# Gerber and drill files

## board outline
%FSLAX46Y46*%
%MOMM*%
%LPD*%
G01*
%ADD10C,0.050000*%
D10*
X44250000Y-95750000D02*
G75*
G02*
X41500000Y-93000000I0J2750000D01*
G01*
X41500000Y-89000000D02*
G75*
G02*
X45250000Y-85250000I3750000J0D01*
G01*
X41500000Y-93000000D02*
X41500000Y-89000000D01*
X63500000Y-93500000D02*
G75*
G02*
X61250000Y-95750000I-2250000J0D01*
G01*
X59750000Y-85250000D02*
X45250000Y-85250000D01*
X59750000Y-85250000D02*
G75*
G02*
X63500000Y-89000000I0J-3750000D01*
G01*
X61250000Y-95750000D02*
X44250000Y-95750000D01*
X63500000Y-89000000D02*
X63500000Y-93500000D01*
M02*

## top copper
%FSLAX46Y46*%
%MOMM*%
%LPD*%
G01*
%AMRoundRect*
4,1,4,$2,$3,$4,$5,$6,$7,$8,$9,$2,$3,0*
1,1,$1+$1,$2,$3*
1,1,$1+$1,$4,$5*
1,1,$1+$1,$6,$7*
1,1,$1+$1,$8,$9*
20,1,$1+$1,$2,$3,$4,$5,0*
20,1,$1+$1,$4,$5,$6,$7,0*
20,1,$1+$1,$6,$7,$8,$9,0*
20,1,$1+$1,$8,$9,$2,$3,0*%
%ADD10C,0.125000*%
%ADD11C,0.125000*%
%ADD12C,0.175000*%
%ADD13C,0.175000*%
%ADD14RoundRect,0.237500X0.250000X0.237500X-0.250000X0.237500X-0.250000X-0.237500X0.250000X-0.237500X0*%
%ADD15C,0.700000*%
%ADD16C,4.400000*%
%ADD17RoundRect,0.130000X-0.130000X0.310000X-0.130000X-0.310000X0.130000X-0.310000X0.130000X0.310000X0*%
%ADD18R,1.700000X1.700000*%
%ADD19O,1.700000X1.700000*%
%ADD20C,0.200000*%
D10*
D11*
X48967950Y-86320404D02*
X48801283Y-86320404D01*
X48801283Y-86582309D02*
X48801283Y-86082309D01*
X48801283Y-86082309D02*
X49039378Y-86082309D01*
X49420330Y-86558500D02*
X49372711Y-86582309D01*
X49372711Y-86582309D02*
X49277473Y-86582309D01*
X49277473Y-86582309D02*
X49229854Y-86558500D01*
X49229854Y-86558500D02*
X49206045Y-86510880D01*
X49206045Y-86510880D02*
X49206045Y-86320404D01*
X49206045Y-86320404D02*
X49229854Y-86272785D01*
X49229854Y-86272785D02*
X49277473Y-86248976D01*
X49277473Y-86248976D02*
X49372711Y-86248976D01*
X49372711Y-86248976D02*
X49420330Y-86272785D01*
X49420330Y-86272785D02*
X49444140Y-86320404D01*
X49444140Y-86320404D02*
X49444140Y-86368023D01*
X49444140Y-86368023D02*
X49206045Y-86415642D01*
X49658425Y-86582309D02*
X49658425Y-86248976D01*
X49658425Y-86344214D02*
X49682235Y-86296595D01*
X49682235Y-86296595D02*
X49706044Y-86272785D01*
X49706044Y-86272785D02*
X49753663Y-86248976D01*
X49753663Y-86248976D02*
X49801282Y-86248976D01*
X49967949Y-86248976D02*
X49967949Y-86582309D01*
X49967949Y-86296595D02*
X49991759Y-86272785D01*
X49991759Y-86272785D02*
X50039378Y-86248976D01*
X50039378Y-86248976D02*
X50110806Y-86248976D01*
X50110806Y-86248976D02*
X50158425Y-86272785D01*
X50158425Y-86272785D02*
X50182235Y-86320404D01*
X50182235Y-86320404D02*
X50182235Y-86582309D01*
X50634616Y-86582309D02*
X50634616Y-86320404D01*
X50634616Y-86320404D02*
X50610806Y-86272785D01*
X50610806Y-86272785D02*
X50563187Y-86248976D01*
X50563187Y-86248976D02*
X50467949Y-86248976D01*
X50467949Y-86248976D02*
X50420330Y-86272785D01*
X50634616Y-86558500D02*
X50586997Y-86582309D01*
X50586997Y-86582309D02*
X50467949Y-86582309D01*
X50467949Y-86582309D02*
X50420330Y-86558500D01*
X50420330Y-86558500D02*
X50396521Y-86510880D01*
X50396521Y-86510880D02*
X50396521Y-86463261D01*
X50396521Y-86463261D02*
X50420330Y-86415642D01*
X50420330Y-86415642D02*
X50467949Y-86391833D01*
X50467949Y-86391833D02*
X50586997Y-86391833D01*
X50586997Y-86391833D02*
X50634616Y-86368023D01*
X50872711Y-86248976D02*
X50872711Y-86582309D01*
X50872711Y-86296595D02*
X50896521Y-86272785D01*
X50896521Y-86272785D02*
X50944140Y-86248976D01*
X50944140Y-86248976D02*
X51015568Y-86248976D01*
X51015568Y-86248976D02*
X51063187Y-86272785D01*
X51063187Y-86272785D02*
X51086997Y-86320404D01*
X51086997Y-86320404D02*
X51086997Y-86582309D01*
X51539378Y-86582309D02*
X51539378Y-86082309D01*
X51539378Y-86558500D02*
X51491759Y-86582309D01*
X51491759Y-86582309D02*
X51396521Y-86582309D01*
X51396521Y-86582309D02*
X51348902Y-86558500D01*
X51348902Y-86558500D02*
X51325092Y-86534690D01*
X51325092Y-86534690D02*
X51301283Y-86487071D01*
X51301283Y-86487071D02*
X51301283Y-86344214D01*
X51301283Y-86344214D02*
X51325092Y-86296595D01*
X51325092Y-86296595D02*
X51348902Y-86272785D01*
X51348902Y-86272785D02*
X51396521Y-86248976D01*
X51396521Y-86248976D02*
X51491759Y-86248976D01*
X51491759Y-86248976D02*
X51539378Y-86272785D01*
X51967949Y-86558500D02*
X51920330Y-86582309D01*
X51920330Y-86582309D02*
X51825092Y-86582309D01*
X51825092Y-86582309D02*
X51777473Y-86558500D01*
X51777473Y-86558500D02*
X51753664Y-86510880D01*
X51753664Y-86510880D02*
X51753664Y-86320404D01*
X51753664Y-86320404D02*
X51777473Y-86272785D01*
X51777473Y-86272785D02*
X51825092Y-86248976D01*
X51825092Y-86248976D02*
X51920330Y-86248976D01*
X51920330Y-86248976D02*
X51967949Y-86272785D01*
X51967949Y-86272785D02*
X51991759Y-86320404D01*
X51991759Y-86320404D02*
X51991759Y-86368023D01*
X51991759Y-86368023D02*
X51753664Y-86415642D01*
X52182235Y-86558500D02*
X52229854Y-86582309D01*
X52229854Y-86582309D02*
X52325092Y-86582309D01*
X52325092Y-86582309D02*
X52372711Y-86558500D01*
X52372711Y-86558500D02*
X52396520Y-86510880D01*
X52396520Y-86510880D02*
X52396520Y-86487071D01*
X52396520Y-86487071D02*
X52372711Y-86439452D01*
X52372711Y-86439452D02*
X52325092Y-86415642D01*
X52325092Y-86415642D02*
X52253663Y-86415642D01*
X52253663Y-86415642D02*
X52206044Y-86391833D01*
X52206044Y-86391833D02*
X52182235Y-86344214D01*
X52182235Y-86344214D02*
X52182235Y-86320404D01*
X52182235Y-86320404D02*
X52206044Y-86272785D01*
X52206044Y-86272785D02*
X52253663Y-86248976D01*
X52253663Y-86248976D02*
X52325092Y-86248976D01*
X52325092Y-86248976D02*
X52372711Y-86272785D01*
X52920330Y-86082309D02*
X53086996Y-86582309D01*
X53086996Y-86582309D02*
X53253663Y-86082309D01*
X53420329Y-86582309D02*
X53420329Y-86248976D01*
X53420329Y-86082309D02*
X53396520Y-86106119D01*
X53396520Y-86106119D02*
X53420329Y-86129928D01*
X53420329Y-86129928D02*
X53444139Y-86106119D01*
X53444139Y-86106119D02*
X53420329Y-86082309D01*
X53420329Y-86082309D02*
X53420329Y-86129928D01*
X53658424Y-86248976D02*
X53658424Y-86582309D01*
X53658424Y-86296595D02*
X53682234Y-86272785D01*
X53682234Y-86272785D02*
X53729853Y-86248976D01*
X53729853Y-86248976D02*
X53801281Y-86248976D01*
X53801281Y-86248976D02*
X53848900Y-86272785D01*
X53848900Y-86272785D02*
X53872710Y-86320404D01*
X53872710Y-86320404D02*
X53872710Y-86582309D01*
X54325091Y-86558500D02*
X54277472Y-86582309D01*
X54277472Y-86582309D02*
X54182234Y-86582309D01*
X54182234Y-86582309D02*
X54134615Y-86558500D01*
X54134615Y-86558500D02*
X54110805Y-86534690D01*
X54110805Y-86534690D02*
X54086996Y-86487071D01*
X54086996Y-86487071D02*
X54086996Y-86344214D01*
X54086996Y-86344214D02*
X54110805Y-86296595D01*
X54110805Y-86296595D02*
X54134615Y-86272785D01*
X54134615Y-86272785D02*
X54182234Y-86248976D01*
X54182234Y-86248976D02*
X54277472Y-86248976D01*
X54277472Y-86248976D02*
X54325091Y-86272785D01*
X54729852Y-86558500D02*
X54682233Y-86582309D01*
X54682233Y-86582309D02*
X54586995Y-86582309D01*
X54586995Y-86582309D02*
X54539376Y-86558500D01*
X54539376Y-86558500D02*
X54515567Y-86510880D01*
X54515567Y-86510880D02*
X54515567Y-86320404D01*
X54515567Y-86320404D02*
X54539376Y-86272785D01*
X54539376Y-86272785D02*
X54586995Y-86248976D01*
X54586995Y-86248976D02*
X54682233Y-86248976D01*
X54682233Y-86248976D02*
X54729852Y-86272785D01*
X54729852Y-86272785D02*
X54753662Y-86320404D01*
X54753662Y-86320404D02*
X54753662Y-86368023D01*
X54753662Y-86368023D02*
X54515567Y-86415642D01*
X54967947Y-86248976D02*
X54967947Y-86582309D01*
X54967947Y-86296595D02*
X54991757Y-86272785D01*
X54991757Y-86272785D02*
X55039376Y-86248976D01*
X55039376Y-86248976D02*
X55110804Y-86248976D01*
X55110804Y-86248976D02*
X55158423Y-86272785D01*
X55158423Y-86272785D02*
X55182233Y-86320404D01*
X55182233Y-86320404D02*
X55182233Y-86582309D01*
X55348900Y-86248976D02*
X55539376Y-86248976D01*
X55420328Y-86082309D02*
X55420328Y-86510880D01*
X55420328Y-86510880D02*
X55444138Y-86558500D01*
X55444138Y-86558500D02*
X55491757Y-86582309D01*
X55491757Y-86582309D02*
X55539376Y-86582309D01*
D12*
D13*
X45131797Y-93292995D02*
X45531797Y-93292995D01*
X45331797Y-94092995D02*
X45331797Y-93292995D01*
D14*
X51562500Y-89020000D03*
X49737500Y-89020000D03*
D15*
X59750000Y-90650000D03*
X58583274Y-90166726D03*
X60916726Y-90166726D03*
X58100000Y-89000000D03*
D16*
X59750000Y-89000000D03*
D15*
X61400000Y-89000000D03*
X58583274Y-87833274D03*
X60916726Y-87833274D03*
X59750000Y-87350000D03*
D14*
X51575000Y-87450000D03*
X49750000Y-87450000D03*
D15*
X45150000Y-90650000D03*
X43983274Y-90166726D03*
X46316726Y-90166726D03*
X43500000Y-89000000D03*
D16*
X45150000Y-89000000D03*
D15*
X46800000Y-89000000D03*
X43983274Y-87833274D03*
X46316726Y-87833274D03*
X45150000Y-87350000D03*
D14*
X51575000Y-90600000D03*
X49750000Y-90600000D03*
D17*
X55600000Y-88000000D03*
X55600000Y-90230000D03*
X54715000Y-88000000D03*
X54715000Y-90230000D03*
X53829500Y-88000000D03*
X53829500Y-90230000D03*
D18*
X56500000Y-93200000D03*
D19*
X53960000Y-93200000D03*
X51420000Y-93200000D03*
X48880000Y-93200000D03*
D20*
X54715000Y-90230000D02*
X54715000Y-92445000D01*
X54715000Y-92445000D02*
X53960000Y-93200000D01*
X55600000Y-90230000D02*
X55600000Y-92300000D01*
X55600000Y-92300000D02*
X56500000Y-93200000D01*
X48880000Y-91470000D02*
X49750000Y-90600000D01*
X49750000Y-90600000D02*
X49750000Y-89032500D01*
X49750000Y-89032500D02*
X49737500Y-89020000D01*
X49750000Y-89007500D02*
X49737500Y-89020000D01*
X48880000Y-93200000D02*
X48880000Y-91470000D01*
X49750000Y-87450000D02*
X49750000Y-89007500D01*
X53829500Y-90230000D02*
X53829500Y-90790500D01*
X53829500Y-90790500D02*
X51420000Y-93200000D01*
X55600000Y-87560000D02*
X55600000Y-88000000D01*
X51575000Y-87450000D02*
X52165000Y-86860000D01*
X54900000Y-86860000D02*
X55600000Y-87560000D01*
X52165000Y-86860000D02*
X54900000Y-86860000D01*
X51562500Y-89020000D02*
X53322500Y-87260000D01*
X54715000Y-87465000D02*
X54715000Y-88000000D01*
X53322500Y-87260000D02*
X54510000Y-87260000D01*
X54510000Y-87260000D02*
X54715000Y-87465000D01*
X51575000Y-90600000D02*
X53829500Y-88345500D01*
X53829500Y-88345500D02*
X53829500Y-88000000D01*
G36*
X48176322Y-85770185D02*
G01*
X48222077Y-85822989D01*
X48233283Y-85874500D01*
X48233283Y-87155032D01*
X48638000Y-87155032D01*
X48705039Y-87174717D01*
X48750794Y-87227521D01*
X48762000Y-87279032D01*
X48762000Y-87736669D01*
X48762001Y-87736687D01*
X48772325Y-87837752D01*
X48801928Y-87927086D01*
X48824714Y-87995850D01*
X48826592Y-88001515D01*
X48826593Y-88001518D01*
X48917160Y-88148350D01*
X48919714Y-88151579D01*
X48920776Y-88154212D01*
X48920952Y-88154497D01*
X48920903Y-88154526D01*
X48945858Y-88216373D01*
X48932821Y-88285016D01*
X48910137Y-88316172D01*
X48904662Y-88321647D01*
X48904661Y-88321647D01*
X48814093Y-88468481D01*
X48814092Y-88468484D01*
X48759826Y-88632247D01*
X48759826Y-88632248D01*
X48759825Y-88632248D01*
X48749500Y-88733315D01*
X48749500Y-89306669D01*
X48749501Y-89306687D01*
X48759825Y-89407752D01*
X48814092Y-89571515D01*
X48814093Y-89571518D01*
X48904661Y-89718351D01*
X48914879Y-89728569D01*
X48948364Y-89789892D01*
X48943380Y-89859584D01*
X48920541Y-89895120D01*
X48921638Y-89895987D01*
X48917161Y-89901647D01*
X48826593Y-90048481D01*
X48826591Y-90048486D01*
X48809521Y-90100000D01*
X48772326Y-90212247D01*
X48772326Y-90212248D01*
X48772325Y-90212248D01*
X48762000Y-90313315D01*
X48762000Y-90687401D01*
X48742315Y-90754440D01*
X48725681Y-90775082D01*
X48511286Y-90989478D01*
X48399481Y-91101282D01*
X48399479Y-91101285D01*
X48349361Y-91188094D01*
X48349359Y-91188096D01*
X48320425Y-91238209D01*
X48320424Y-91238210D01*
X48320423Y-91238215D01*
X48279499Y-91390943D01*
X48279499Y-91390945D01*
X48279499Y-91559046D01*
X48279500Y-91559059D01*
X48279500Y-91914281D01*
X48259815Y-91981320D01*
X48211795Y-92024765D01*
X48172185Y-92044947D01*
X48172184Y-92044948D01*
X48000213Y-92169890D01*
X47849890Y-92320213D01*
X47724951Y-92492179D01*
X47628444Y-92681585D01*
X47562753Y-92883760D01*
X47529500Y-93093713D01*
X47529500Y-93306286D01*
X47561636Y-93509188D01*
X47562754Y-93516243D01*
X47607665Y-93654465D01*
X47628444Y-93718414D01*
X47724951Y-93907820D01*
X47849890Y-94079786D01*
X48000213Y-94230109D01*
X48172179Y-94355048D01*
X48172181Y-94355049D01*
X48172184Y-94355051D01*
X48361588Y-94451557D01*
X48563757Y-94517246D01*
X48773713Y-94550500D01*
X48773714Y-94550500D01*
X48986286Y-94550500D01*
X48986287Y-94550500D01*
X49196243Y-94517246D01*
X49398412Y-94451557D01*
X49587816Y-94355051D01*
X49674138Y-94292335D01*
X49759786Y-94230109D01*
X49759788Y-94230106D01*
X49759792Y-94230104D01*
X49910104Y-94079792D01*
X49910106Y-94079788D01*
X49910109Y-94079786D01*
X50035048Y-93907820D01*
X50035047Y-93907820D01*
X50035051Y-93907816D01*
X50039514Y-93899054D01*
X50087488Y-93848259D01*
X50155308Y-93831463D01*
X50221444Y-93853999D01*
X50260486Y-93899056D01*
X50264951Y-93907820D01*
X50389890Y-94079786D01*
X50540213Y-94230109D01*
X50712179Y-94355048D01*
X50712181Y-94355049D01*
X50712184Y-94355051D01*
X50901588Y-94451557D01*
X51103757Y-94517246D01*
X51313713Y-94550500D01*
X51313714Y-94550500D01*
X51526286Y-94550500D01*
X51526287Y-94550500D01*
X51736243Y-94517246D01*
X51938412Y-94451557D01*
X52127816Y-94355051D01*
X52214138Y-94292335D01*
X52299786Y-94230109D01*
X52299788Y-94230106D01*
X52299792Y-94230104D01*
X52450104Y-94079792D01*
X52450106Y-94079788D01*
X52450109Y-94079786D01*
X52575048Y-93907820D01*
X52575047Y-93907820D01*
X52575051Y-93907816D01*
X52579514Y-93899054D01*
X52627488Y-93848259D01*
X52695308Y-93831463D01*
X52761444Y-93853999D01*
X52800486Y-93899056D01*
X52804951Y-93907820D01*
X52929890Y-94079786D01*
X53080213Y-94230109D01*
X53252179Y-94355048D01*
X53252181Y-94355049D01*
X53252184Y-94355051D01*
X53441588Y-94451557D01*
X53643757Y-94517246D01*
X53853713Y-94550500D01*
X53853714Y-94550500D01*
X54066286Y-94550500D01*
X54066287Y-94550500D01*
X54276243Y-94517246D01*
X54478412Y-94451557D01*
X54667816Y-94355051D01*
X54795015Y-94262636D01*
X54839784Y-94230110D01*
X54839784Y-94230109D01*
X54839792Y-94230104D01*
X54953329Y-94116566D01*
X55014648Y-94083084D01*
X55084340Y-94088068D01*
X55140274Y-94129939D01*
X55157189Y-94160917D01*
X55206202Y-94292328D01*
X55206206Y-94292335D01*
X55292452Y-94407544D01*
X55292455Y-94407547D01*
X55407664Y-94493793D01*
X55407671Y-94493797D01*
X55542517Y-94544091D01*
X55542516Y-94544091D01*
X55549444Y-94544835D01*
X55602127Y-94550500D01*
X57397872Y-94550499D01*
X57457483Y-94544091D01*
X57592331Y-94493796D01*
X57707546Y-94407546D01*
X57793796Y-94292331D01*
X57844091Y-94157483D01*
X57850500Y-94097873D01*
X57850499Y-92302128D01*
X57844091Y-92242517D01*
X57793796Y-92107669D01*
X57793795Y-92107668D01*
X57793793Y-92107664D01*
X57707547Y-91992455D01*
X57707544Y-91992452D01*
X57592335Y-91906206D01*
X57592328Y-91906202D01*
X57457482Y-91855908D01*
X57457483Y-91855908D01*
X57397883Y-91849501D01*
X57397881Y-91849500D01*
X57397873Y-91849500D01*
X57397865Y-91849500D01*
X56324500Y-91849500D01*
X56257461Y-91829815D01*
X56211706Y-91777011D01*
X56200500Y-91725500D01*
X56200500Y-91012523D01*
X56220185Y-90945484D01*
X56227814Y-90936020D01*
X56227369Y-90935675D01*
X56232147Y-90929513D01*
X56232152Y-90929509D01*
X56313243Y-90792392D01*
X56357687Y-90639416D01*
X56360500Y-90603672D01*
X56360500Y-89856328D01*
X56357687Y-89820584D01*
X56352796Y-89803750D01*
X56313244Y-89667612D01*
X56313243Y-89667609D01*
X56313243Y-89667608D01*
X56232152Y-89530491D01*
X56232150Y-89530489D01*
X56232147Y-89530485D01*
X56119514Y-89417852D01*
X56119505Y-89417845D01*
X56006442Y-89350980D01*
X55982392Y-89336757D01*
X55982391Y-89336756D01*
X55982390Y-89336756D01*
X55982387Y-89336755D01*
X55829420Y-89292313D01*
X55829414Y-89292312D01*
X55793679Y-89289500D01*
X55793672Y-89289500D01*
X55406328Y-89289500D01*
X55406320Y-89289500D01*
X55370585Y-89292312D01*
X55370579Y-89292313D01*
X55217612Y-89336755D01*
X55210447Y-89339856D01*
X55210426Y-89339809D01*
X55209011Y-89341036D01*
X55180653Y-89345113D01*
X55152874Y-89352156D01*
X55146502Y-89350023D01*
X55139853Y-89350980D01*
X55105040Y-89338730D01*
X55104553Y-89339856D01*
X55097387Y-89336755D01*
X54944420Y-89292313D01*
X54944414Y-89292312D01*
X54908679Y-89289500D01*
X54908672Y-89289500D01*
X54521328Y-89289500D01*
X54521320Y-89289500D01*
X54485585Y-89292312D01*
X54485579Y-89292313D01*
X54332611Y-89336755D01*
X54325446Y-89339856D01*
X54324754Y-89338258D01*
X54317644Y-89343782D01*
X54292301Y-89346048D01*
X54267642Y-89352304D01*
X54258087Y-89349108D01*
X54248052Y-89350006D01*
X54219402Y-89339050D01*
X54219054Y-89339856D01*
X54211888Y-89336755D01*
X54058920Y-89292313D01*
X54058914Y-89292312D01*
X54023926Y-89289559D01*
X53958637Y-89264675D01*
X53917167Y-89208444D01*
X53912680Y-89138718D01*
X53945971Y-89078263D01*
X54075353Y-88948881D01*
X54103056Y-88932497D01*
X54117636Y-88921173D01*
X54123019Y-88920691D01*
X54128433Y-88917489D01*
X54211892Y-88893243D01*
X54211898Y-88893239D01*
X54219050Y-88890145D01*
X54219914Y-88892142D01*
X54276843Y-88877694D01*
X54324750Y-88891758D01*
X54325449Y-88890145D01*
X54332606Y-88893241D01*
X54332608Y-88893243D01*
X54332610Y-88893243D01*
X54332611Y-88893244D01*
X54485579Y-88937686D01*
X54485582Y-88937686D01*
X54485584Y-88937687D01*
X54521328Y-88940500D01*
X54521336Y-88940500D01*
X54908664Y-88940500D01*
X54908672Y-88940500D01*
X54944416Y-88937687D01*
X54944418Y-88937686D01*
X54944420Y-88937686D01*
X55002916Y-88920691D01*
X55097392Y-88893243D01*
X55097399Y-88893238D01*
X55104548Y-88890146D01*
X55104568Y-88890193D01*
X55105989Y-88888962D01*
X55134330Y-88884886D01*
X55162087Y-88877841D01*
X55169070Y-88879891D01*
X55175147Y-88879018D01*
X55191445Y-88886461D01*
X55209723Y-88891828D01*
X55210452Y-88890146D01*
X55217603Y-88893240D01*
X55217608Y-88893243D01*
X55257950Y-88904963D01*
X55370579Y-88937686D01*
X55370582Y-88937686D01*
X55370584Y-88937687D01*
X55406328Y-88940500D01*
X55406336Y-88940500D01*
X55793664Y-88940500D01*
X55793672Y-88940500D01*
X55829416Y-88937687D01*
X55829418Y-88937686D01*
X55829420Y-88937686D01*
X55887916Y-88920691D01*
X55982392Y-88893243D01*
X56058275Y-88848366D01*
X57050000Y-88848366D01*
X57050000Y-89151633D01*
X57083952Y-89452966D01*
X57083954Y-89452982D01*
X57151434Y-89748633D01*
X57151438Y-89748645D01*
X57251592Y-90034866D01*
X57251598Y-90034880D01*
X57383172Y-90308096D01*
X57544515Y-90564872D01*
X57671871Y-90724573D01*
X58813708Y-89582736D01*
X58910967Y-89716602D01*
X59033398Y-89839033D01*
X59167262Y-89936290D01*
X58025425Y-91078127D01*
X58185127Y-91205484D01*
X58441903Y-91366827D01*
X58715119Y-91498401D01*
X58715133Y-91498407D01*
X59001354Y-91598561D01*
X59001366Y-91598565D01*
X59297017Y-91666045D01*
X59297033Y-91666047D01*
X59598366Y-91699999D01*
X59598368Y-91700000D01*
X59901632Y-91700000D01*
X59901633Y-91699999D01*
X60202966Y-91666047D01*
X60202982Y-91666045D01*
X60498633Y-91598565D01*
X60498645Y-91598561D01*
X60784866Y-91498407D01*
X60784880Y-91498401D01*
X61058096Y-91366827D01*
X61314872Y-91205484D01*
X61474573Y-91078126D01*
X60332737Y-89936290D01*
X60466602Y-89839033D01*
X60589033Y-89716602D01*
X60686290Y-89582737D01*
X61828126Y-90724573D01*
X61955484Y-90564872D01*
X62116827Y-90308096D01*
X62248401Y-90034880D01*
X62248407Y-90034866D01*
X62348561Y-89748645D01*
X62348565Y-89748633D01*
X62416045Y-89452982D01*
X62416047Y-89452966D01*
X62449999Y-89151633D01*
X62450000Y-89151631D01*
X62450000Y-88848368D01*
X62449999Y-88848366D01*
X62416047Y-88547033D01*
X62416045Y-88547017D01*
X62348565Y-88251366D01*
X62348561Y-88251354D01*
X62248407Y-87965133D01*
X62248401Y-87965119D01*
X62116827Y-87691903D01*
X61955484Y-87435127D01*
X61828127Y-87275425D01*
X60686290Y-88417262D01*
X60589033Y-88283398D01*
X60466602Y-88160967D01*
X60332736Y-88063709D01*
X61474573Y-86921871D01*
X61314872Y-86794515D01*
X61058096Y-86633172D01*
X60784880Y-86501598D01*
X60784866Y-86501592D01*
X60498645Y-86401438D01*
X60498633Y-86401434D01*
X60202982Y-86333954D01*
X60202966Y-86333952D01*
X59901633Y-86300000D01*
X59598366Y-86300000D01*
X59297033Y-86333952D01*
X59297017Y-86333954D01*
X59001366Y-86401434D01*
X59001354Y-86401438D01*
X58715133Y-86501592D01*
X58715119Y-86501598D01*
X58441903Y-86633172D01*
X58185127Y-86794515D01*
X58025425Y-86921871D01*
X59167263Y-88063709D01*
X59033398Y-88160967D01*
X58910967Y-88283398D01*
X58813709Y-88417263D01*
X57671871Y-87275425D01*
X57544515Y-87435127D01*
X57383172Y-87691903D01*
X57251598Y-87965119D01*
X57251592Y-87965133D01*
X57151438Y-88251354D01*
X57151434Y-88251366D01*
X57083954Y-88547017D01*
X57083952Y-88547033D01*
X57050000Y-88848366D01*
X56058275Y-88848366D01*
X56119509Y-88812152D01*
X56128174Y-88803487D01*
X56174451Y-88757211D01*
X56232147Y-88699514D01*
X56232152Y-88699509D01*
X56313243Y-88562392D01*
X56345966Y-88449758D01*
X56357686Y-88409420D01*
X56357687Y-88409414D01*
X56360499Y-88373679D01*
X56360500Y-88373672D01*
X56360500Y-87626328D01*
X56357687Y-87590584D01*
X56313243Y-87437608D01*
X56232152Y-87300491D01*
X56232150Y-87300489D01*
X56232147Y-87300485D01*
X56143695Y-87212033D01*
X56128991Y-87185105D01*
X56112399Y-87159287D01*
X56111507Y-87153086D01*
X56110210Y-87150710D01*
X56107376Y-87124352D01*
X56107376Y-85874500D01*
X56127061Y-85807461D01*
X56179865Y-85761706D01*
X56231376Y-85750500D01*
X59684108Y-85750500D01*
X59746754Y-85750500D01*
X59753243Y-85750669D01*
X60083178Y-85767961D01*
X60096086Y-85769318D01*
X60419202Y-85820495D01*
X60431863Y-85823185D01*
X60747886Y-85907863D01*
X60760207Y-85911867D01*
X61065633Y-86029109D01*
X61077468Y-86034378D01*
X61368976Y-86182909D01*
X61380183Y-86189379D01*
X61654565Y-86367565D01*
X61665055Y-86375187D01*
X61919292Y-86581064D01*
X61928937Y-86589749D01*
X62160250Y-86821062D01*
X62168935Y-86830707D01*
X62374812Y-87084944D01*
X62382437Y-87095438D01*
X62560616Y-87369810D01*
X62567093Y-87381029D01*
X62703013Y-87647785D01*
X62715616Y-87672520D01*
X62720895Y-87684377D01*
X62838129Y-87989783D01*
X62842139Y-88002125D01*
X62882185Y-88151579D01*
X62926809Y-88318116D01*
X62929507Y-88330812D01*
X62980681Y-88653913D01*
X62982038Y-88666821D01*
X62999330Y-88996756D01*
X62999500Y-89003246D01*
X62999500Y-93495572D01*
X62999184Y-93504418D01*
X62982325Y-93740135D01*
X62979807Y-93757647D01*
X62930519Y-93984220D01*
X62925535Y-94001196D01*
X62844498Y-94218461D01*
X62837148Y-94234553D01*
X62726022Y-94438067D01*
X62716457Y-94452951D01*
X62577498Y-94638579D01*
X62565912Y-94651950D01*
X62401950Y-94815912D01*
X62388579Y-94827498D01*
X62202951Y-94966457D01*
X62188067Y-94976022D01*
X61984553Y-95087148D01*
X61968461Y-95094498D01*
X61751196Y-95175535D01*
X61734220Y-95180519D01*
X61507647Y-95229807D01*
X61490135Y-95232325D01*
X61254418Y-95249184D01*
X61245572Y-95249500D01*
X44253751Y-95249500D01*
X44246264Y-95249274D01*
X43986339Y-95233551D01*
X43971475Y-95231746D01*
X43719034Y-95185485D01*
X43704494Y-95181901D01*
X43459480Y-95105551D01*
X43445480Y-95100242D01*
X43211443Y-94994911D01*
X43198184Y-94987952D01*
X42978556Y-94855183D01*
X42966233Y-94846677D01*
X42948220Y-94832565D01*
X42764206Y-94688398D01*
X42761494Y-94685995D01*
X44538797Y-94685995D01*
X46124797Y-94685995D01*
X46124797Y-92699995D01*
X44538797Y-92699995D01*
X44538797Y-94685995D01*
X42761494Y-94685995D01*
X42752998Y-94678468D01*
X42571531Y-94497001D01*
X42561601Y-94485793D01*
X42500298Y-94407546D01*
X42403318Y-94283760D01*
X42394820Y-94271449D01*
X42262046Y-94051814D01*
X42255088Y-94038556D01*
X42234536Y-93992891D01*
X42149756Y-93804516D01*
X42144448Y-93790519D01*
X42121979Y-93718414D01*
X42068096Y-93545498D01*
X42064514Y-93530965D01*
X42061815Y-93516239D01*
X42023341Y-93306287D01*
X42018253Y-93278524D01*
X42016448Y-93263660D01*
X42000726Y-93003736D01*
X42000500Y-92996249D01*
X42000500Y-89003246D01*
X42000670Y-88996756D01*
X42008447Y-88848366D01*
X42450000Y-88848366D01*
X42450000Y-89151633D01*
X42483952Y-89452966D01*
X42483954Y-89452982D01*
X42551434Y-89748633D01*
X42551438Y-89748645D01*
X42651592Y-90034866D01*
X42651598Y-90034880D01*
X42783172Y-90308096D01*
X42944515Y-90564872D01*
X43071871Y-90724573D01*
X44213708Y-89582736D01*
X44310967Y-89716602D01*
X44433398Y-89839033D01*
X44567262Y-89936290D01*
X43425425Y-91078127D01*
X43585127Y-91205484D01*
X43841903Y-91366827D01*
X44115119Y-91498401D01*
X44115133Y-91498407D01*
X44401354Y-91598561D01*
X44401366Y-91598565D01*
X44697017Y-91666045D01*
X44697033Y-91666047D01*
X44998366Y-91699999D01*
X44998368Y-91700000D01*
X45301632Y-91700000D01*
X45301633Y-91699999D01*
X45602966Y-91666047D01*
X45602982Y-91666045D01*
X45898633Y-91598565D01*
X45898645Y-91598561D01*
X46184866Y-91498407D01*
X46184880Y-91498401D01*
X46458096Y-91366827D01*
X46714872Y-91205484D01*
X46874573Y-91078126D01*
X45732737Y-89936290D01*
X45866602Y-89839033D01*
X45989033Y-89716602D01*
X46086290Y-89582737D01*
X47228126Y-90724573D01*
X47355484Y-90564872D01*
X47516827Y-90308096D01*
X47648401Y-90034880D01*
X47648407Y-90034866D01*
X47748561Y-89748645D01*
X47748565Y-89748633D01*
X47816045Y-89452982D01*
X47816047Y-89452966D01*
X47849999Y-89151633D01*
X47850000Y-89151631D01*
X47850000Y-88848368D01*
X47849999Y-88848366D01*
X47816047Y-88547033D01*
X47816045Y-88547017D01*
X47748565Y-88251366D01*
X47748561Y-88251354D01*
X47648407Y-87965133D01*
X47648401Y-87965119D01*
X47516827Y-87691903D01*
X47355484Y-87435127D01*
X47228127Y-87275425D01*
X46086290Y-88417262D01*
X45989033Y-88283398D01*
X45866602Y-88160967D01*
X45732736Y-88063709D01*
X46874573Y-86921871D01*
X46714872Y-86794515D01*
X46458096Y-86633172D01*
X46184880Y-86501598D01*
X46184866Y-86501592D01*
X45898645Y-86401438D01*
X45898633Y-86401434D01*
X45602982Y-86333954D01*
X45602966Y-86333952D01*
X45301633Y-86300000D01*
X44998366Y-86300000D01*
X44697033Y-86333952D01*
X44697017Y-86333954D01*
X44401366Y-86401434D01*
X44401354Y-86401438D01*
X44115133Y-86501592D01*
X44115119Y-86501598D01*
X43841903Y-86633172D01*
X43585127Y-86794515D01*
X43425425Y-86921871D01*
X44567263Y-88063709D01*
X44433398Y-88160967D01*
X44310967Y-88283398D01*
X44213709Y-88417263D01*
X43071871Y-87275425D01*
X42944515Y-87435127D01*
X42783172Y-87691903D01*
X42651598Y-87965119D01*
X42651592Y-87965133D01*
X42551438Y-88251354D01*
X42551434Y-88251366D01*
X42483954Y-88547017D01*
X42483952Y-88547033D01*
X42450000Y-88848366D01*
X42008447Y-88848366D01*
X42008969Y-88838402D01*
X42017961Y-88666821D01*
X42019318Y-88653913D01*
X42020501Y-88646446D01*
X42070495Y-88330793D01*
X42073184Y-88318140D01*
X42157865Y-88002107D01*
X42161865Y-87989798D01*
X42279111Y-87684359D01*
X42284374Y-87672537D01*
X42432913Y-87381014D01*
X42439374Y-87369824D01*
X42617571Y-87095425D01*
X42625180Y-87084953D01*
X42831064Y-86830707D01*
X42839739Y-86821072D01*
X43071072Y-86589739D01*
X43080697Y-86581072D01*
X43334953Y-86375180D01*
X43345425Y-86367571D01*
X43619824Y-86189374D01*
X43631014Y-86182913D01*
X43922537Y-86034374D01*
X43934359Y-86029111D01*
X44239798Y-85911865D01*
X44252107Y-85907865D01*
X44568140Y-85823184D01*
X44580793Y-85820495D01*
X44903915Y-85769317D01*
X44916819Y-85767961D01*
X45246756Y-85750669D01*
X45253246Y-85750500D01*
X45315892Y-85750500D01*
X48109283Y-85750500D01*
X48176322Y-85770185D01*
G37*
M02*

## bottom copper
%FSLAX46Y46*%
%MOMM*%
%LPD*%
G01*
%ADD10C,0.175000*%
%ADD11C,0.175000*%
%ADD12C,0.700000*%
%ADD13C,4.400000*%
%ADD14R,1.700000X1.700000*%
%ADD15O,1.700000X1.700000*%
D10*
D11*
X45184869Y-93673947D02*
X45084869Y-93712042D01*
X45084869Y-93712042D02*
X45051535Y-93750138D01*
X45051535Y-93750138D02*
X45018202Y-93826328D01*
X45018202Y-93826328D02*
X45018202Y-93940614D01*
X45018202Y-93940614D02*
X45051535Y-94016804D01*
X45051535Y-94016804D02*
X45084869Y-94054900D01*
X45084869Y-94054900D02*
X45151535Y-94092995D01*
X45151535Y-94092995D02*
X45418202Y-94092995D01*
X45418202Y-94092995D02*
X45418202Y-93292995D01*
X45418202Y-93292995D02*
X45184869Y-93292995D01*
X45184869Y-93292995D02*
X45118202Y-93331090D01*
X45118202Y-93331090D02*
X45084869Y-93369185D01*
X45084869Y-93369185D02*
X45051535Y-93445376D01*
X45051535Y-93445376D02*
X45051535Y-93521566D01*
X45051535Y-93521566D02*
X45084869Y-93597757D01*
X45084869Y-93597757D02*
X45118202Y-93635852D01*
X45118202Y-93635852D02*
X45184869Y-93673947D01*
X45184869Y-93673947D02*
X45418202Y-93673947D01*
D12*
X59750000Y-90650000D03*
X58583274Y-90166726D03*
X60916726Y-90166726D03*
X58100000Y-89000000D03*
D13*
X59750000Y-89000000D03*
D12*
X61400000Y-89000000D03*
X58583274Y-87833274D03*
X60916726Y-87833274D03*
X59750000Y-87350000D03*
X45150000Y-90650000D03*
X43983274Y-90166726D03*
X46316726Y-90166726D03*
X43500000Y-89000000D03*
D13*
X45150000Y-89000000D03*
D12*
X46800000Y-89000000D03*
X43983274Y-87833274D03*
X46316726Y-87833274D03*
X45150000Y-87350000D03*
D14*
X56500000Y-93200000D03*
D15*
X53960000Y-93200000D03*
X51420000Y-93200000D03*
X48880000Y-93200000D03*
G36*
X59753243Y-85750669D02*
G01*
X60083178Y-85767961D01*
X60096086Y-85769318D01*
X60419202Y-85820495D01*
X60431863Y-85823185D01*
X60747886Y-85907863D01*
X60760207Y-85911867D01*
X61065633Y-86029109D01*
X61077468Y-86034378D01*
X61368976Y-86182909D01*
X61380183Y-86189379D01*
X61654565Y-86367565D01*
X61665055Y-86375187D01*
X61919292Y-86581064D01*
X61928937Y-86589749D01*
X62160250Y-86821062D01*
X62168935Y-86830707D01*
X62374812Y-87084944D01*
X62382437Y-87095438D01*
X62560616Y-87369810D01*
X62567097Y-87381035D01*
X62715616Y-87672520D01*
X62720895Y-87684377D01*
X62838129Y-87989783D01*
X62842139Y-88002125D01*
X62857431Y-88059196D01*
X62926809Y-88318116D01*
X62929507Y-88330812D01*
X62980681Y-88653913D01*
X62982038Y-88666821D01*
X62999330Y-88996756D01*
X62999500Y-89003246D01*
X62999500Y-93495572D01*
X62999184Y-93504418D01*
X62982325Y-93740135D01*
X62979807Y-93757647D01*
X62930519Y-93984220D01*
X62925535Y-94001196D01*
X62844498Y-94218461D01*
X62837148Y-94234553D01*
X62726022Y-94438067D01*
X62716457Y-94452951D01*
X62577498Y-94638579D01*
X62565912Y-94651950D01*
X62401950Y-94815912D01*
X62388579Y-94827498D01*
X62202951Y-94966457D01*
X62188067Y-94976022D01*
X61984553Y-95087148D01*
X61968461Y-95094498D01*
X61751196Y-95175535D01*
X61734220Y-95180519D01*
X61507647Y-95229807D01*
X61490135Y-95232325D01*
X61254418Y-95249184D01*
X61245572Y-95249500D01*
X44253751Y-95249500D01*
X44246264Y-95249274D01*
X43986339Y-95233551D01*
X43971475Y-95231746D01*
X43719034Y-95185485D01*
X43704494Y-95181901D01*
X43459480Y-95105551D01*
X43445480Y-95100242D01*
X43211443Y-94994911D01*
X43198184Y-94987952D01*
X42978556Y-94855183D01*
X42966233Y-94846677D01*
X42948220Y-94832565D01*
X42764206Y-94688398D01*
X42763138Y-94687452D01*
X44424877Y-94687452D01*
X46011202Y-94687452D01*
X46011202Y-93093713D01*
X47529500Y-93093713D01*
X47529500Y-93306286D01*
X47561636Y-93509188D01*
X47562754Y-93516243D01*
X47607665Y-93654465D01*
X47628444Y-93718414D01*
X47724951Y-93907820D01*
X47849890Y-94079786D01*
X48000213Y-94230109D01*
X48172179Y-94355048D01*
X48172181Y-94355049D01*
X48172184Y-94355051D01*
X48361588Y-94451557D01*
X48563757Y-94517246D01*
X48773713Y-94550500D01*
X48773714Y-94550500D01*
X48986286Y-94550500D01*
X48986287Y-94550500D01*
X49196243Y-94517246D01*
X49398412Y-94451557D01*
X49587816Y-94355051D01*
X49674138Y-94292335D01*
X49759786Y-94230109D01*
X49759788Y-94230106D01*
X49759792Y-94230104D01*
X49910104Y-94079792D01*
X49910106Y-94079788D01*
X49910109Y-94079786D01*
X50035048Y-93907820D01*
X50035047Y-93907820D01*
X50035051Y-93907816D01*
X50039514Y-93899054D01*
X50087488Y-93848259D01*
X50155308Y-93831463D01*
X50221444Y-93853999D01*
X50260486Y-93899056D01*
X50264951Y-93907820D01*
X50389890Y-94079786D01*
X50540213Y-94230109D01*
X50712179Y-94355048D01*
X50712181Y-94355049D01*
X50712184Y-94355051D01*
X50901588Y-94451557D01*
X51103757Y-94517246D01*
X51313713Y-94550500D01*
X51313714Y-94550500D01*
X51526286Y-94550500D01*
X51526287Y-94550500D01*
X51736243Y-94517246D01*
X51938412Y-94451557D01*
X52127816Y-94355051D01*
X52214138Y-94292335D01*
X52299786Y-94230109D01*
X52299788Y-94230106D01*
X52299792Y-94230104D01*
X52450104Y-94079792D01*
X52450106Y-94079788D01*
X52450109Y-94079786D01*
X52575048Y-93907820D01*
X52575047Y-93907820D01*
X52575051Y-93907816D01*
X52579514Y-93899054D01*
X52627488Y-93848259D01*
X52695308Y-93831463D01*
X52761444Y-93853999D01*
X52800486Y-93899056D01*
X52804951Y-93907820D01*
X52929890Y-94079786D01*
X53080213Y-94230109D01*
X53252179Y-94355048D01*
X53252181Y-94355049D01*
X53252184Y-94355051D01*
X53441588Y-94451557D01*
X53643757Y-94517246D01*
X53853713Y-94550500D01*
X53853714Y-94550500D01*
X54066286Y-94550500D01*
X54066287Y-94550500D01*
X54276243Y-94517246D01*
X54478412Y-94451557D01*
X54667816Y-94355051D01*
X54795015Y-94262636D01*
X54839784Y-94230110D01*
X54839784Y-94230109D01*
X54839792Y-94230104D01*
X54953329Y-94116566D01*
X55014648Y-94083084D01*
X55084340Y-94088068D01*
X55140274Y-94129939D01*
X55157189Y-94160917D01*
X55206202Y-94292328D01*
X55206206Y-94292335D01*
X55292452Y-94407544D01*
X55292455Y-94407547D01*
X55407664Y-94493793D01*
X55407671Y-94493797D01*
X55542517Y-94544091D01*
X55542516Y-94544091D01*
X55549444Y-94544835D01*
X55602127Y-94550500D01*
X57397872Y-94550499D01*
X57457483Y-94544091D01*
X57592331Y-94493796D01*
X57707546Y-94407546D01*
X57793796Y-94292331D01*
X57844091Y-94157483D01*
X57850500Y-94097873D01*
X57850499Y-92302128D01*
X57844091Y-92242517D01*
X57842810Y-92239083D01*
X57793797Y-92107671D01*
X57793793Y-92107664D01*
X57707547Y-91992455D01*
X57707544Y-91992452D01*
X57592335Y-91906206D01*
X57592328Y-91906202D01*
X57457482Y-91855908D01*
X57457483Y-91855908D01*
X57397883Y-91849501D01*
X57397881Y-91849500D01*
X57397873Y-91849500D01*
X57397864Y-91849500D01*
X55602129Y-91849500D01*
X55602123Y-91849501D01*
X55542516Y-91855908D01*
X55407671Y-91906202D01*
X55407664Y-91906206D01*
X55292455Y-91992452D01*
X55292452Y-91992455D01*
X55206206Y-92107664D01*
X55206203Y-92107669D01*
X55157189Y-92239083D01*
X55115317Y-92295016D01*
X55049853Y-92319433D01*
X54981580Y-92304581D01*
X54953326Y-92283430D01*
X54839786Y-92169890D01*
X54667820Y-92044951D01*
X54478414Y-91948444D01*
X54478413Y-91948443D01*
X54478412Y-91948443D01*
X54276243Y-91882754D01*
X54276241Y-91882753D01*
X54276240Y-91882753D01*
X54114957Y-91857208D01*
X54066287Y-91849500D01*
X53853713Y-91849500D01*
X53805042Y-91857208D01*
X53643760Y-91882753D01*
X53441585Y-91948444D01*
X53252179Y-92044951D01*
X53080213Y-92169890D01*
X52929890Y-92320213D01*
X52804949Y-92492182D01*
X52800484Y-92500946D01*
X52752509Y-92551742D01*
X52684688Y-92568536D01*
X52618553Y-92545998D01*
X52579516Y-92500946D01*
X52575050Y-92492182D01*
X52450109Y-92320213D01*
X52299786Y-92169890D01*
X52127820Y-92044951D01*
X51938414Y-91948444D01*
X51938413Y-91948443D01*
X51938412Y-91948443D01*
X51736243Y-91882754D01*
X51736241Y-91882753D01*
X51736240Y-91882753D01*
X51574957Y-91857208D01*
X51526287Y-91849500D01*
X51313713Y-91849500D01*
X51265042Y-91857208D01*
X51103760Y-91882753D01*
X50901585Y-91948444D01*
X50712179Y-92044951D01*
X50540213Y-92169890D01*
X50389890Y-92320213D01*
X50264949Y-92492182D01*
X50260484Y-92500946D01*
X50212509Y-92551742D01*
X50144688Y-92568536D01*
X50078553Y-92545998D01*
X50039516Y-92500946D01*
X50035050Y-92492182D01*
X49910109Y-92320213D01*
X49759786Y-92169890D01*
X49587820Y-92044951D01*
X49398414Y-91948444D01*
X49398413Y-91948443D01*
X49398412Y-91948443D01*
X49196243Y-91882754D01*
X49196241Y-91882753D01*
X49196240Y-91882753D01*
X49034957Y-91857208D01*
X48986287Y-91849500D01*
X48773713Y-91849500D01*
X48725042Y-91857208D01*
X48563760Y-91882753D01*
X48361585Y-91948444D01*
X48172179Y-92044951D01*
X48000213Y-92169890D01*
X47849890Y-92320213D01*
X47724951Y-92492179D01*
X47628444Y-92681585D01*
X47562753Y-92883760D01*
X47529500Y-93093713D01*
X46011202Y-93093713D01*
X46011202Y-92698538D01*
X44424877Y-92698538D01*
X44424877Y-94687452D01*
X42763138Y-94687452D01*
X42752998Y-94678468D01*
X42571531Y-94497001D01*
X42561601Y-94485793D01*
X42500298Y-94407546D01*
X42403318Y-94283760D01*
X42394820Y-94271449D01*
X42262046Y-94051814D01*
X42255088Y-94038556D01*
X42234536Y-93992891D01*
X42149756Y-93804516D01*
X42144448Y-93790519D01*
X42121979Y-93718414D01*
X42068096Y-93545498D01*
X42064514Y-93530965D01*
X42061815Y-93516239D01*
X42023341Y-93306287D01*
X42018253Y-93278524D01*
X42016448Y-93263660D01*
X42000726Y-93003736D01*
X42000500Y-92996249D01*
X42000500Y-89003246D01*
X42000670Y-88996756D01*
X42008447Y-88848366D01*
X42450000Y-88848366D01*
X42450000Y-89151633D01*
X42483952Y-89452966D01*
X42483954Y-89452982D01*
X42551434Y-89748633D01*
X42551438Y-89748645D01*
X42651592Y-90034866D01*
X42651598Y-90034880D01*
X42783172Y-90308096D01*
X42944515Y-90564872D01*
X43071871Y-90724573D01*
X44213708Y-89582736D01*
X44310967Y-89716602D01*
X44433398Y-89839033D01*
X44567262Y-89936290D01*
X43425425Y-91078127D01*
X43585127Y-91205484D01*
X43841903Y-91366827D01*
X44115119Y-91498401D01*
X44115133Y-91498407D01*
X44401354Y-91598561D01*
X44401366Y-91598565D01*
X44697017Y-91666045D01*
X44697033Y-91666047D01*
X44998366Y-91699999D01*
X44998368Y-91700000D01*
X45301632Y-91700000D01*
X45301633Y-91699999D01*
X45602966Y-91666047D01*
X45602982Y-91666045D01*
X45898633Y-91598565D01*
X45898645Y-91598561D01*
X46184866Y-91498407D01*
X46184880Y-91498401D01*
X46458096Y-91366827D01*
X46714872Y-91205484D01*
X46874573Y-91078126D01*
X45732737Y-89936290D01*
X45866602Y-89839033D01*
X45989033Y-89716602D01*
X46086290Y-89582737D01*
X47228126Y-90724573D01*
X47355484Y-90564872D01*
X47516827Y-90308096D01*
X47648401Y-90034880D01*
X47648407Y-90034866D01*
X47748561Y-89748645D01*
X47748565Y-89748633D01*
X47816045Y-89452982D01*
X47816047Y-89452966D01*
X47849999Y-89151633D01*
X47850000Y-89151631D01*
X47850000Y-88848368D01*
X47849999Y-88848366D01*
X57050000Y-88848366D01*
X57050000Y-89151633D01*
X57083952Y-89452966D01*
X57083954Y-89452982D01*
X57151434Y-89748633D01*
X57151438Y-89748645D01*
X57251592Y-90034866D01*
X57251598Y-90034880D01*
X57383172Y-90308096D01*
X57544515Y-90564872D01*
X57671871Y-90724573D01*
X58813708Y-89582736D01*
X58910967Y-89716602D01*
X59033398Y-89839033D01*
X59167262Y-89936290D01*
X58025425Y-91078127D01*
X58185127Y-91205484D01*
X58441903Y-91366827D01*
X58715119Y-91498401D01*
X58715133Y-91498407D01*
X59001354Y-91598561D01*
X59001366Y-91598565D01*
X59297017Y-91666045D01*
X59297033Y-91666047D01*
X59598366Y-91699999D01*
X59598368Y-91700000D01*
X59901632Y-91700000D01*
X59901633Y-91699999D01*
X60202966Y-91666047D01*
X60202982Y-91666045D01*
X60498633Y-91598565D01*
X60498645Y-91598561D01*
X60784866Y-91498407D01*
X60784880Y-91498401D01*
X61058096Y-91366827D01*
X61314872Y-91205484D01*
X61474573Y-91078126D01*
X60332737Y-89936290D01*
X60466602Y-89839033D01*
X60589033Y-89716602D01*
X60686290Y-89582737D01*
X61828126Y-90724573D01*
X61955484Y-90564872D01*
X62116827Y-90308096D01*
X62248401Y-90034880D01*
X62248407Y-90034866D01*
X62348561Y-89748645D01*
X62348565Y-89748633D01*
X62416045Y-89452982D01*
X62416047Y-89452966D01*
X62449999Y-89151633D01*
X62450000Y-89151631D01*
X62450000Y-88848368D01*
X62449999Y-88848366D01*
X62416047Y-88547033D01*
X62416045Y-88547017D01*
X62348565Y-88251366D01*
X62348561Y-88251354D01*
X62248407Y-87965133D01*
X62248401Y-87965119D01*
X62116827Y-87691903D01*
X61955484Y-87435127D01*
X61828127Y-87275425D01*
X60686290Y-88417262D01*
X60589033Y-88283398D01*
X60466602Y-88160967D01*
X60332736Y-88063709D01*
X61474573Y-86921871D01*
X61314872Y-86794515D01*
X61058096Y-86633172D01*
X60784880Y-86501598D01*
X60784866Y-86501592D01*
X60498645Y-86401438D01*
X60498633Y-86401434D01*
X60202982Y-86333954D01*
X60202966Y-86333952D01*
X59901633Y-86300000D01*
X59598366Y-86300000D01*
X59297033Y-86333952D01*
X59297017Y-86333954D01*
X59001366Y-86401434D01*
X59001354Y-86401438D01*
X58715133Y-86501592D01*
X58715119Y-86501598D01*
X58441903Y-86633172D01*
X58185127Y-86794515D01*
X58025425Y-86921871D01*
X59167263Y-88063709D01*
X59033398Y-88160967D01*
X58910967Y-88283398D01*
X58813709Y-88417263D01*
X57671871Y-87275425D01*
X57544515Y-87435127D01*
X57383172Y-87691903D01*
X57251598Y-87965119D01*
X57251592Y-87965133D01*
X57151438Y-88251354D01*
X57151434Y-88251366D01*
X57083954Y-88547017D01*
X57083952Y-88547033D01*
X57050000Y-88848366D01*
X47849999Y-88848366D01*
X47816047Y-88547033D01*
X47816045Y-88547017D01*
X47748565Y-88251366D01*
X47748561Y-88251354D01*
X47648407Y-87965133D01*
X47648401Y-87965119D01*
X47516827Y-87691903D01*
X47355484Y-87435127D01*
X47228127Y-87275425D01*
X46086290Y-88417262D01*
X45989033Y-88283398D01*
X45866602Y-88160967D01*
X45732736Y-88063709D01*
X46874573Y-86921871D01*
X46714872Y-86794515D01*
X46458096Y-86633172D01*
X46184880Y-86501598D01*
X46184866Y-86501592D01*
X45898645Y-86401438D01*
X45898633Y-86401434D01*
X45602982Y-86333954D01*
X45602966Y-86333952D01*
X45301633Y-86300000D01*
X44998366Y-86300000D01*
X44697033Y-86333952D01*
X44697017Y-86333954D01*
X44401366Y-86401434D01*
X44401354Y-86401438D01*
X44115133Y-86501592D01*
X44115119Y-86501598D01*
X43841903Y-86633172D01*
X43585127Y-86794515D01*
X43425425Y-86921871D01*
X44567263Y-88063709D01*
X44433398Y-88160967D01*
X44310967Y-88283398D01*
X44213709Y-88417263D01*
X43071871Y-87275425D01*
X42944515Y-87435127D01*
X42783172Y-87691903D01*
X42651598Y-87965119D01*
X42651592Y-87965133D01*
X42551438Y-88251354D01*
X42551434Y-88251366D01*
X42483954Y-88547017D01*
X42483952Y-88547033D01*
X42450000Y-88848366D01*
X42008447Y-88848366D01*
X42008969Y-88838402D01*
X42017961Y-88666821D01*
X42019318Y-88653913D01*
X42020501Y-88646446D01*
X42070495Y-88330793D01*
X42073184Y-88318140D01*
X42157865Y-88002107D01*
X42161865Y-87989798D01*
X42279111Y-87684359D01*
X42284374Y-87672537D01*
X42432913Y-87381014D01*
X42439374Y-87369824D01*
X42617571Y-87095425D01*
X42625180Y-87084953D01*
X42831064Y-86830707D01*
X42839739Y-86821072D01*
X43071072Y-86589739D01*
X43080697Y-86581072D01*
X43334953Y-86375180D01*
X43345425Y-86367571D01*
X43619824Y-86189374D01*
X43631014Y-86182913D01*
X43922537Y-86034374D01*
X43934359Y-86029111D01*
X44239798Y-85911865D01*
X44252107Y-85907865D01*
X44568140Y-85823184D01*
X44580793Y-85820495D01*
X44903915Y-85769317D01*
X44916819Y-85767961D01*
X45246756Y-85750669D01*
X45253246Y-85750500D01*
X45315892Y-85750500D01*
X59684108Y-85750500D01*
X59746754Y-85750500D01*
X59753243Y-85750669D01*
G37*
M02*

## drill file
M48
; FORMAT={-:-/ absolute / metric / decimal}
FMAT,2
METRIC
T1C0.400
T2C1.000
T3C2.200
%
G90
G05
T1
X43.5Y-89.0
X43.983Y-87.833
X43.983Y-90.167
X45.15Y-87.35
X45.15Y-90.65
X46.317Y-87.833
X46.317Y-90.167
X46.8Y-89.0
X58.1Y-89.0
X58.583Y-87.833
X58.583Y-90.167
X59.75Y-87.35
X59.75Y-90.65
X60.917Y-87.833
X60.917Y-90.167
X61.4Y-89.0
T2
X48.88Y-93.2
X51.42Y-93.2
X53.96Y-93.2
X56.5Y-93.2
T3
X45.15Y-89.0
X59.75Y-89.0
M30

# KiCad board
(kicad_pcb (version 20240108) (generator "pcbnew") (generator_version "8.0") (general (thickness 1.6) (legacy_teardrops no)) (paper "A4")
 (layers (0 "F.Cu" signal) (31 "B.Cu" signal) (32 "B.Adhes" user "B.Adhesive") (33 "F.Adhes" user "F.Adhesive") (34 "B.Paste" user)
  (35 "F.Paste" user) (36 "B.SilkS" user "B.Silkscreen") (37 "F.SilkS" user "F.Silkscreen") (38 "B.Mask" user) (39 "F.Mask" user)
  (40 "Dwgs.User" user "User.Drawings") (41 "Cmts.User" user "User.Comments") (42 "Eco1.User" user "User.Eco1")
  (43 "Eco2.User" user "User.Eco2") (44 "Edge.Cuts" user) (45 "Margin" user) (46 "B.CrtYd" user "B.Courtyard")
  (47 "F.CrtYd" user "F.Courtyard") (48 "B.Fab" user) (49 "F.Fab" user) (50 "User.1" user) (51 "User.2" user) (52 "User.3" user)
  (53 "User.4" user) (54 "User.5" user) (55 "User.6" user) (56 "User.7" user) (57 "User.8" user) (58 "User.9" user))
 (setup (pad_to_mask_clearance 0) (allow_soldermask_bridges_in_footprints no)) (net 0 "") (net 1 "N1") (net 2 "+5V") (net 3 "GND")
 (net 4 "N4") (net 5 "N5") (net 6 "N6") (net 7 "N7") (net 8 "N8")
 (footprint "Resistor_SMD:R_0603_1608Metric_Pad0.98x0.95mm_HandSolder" (layer "F.Cu") (at 50.65 89.02 180)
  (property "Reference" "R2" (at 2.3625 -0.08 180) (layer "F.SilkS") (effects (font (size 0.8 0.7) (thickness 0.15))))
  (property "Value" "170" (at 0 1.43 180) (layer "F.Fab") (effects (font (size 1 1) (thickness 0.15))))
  (pad "1" smd roundrect (at -0.9125 0 180) (size 0.975 0.95) (layers "F.Cu" "F.Paste" "F.Mask") (roundrect_rratio 0.25) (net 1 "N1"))
  (pad "2" smd roundrect (at 0.9125 0 180) (size 0.975 0.95) (layers "F.Cu" "F.Paste" "F.Mask") (roundrect_rratio 0.25) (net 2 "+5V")))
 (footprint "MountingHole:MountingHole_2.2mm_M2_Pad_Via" (layer "F.Cu") (at 59.75 89 90)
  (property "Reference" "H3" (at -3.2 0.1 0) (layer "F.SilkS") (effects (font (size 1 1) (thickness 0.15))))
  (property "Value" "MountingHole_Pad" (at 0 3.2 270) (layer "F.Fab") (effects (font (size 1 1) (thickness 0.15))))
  (pad "1" thru_hole circle (at -1.65 0 90) (size 0.7 0.7) (drill 0.4) (layers "*.Cu" "*.Mask") (remove_unused_layers no) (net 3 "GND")
   (zone_connect 2))
  (pad "1" thru_hole circle (at -1.166726 -1.166726 90) (size 0.7 0.7) (drill 0.4) (layers "*.Cu" "*.Mask") (remove_unused_layers no)
   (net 3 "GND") (zone_connect 2))
  (pad "1" thru_hole circle (at -1.166726 1.166726 90) (size 0.7 0.7) (drill 0.4) (layers "*.Cu" "*.Mask") (remove_unused_layers no)
   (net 3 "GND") (zone_connect 2))
  (pad "1" thru_hole circle (at 0 -1.65 90) (size 0.7 0.7) (drill 0.4) (layers "*.Cu" "*.Mask") (remove_unused_layers no) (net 3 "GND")
   (zone_connect 2))
  (pad "1" thru_hole circle (at 0 0 90) (size 4.4 4.4) (drill 2.2) (layers "*.Cu" "*.Mask") (remove_unused_layers no) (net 3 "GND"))
  (pad "1" thru_hole circle (at 0 1.65 90) (size 0.7 0.7) (drill 0.4) (layers "*.Cu" "*.Mask") (remove_unused_layers no) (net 3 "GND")
   (zone_connect 2))
  (pad "1" thru_hole circle (at 1.166726 -1.166726 90) (size 0.7 0.7) (drill 0.4) (layers "*.Cu" "*.Mask") (remove_unused_layers no)
   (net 3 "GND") (zone_connect 2))
  (pad "1" thru_hole circle (at 1.166726 1.166726 90) (size 0.7 0.7) (drill 0.4) (layers "*.Cu" "*.Mask") (remove_unused_layers no)
   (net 3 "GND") (zone_connect 2))
  (pad "1" thru_hole circle (at 1.65 0 90) (size 0.7 0.7) (drill 0.4) (layers "*.Cu" "*.Mask") (remove_unused_layers no) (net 3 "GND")
   (zone_connect 2)))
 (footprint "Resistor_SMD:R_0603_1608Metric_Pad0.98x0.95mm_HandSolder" (layer "F.Cu") (at 50.6625 87.45 180)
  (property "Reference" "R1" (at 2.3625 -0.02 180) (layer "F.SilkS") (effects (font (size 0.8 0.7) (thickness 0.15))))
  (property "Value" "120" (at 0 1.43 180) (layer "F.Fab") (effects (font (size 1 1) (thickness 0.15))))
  (pad "1" smd roundrect (at -0.9125 0 180) (size 0.975 0.95) (layers "F.Cu" "F.Paste" "F.Mask") (roundrect_rratio 0.25) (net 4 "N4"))
  (pad "2" smd roundrect (at 0.9125 0 180) (size 0.975 0.95) (layers "F.Cu" "F.Paste" "F.Mask") (roundrect_rratio 0.25) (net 2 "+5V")))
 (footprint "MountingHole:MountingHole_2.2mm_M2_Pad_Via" (layer "F.Cu") (at 45.15 89 90)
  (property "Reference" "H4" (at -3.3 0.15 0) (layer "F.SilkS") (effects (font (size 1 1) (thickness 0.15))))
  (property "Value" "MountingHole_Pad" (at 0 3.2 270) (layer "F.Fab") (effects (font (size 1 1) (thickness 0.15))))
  (pad "1" thru_hole circle (at -1.65 0 90) (size 0.7 0.7) (drill 0.4) (layers "*.Cu" "*.Mask") (remove_unused_layers no) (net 3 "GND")
   (zone_connect 2))
  (pad "1" thru_hole circle (at -1.166726 -1.166726 90) (size 0.7 0.7) (drill 0.4) (layers "*.Cu" "*.Mask") (remove_unused_layers no)
   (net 3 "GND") (zone_connect 2))
  (pad "1" thru_hole circle (at -1.166726 1.166726 90) (size 0.7 0.7) (drill 0.4) (layers "*.Cu" "*.Mask") (remove_unused_layers no)
   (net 3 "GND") (zone_connect 2))
  (pad "1" thru_hole circle (at 0 -1.65 90) (size 0.7 0.7) (drill 0.4) (layers "*.Cu" "*.Mask") (remove_unused_layers no) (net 3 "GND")
   (zone_connect 2))
  (pad "1" thru_hole circle (at 0 0 90) (size 4.4 4.4) (drill 2.2) (layers "*.Cu" "*.Mask") (remove_unused_layers no) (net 3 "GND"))
  (pad "1" thru_hole circle (at 0 1.65 90) (size 0.7 0.7) (drill 0.4) (layers "*.Cu" "*.Mask") (remove_unused_layers no) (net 3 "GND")
   (zone_connect 2))
  (pad "1" thru_hole circle (at 1.166726 -1.166726 90) (size 0.7 0.7) (drill 0.4) (layers "*.Cu" "*.Mask") (remove_unused_layers no)
   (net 3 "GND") (zone_connect 2))
  (pad "1" thru_hole circle (at 1.166726 1.166726 90) (size 0.7 0.7) (drill 0.4) (layers "*.Cu" "*.Mask") (remove_unused_layers no)
   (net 3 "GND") (zone_connect 2))
  (pad "1" thru_hole circle (at 1.65 0 90) (size 0.7 0.7) (drill 0.4) (layers "*.Cu" "*.Mask") (remove_unused_layers no) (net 3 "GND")
   (zone_connect 2)))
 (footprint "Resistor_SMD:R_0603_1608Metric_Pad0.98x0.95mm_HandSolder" (layer "F.Cu") (at 50.6625 90.6 180)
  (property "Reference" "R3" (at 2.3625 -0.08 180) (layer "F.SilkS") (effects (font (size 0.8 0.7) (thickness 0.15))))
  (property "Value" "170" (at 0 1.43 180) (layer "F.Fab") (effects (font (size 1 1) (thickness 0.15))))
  (pad "1" smd roundrect (at -0.9125 0 180) (size 0.975 0.95) (layers "F.Cu" "F.Paste" "F.Mask") (roundrect_rratio 0.25) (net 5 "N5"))
  (pad "2" smd roundrect (at 0.9125 0 180) (size 0.975 0.95) (layers "F.Cu" "F.Paste" "F.Mask") (roundrect_rratio 0.25) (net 2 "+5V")))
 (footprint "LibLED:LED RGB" (layer "F.Cu") (at 55.6 88 -90)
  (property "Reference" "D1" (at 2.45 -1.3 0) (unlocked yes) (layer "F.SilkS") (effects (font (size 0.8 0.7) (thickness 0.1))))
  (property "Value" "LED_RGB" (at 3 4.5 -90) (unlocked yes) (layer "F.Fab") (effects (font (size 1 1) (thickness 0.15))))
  (pad "1" smd roundrect (at 0 0 270) (size 0.88 0.52) (layers "F.Cu" "F.Paste" "F.Mask") (roundrect_rratio 0.25) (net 4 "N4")
   (thermal_bridge_angle 45))
  (pad "2" smd roundrect (at 2.23 0 270) (size 0.88 0.52) (layers "F.Cu" "F.Paste" "F.Mask") (roundrect_rratio 0.25) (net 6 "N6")
   (thermal_bridge_angle 45))
  (pad "3" smd roundrect (at 0 0.885 270) (size 0.88 0.52) (layers "F.Cu" "F.Paste" "F.Mask") (roundrect_rratio 0.25) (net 1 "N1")
   (thermal_bridge_angle 45))
  (pad "4" smd roundrect (at 2.23 0.885 270) (size 0.88 0.52) (layers "F.Cu" "F.Paste" "F.Mask") (roundrect_rratio 0.25) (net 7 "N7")
   (thermal_bridge_angle 45))
  (pad "5" smd roundrect (at 0 1.7705 270) (size 0.88 0.52) (layers "F.Cu" "F.Paste" "F.Mask") (roundrect_rratio 0.25) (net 5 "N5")
   (thermal_bridge_angle 45))
  (pad "6" smd roundrect (at 2.23 1.7705 270) (size 0.88 0.52) (layers "F.Cu" "F.Paste" "F.Mask") (roundrect_rratio 0.25) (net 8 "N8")
   (thermal_bridge_angle 45)))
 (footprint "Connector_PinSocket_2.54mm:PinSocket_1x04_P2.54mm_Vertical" (layer "B.Cu") (at 56.5 93.2 90)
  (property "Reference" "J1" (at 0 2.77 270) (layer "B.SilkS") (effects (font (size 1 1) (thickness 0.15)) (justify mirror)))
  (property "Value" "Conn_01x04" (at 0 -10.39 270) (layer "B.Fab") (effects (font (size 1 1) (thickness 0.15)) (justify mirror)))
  (pad "1" thru_hole rect (at 0 0 90) (size 1.7 1.7) (drill 1) (layers "*.Cu" "*.Mask") (remove_unused_layers no) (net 6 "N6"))
  (pad "2" thru_hole oval (at 0 -2.54 90) (size 1.7 1.7) (drill 1) (layers "*.Cu" "*.Mask") (remove_unused_layers no) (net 7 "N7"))
  (pad "3" thru_hole oval (at 0 -5.08 90) (size 1.7 1.7) (drill 1) (layers "*.Cu" "*.Mask") (remove_unused_layers no) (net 8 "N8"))
  (pad "4" thru_hole oval (at 0 -7.62 90) (size 1.7 1.7) (drill 1) (layers "*.Cu" "*.Mask") (remove_unused_layers no) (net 2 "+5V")))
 (gr_arc (start 44.25 95.75) (mid 42.305456 94.944544) (end 41.5 93) (stroke (width 0.05) (type default)) (layer "Edge.Cuts"))
 (gr_arc (start 41.5 89) (mid 42.59835 86.34835) (end 45.25 85.25) (stroke (width 0.05) (type default)) (layer "Edge.Cuts"))
 (gr_line (start 41.5 93) (end 41.5 89) (stroke (width 0.05) (type default)) (layer "Edge.Cuts"))
 (gr_arc (start 63.5 93.5) (mid 62.84099 95.09099) (end 61.25 95.75) (stroke (width 0.05) (type default)) (layer "Edge.Cuts"))
 (gr_line (start 59.75 85.25) (end 45.25 85.25) (stroke (width 0.05) (type default)) (layer "Edge.Cuts"))
 (gr_arc (start 59.75 85.25) (mid 62.40165 86.34835) (end 63.5 89) (stroke (width 0.05) (type default)) (layer "Edge.Cuts"))
 (gr_line (start 61.25 95.75) (end 44.25 95.75) (stroke (width 0.05) (type default)) (layer "Edge.Cuts"))
 (gr_line (start 63.5 89) (end 63.5 93.5) (stroke (width 0.05) (type default)) (layer "Edge.Cuts"))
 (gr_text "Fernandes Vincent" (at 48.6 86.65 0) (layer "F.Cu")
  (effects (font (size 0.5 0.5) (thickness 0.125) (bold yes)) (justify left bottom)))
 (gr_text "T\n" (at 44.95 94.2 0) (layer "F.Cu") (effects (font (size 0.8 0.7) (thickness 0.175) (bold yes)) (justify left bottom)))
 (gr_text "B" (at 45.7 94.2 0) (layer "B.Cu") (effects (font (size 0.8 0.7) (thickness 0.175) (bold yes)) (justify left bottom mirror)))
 (segment (start 54.715 90.23) (end 54.715 92.445) (width 0.2) (layer "F.Cu") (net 7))
 (segment (start 54.715 92.445) (end 53.96 93.2) (width 0.2) (layer "F.Cu") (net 7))
 (segment (start 55.6 90.23) (end 55.6 92.3) (width 0.2) (layer "F.Cu") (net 6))
 (segment (start 55.6 92.3) (end 56.5 93.2) (width 0.2) (layer "F.Cu") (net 6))
 (segment (start 48.88 91.47) (end 49.75 90.6) (width 0.2) (layer "F.Cu") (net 2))
 (segment (start 49.75 90.6) (end 49.75 89.0325) (width 0.2) (layer "F.Cu") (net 2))
 (segment (start 49.75 89.0325) (end 49.7375 89.02) (width 0.2) (layer "F.Cu") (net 2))
 (segment (start 49.75 89.0075) (end 49.7375 89.02) (width 0.2) (layer "F.Cu") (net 2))
 (segment (start 48.88 93.2) (end 48.88 91.47) (width 0.2) (layer "F.Cu") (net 2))
 (segment (start 49.75 87.45) (end 49.75 89.0075) (width 0.2) (layer "F.Cu") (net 2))
 (segment (start 53.8295 90.23) (end 53.8295 90.7905) (width 0.2) (layer "F.Cu") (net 8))
 (segment (start 53.8295 90.7905) (end 51.42 93.2) (width 0.2) (layer "F.Cu") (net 8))
 (segment (start 55.6 87.56) (end 55.6 88) (width 0.2) (layer "F.Cu") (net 4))
 (segment (start 51.575 87.45) (end 52.165 86.86) (width 0.2) (layer "F.Cu") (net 4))
 (segment (start 54.9 86.86) (end 55.6 87.56) (width 0.2) (layer "F.Cu") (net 4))
 (segment (start 52.165 86.86) (end 54.9 86.86) (width 0.2) (layer "F.Cu") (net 4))
 (segment (start 51.5625 89.02) (end 53.3225 87.26) (width 0.2) (layer "F.Cu") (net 1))
 (segment (start 54.715 87.465) (end 54.715 88) (width 0.2) (layer "F.Cu") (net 1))
 (segment (start 53.3225 87.26) (end 54.51 87.26) (width 0.2) (layer "F.Cu") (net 1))
 (segment (start 54.51 87.26) (end 54.715 87.465) (width 0.2) (layer "F.Cu") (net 1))
 (segment (start 51.575 90.6) (end 53.8295 88.3455) (width 0.2) (layer "F.Cu") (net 5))
 (segment (start 53.8295 88.3455) (end 53.8295 88) (width 0.2) (layer "F.Cu") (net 5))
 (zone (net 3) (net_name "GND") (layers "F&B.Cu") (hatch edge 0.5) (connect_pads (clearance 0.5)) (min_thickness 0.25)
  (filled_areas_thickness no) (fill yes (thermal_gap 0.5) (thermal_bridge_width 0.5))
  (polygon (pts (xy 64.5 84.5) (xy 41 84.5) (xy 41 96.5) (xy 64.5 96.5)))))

